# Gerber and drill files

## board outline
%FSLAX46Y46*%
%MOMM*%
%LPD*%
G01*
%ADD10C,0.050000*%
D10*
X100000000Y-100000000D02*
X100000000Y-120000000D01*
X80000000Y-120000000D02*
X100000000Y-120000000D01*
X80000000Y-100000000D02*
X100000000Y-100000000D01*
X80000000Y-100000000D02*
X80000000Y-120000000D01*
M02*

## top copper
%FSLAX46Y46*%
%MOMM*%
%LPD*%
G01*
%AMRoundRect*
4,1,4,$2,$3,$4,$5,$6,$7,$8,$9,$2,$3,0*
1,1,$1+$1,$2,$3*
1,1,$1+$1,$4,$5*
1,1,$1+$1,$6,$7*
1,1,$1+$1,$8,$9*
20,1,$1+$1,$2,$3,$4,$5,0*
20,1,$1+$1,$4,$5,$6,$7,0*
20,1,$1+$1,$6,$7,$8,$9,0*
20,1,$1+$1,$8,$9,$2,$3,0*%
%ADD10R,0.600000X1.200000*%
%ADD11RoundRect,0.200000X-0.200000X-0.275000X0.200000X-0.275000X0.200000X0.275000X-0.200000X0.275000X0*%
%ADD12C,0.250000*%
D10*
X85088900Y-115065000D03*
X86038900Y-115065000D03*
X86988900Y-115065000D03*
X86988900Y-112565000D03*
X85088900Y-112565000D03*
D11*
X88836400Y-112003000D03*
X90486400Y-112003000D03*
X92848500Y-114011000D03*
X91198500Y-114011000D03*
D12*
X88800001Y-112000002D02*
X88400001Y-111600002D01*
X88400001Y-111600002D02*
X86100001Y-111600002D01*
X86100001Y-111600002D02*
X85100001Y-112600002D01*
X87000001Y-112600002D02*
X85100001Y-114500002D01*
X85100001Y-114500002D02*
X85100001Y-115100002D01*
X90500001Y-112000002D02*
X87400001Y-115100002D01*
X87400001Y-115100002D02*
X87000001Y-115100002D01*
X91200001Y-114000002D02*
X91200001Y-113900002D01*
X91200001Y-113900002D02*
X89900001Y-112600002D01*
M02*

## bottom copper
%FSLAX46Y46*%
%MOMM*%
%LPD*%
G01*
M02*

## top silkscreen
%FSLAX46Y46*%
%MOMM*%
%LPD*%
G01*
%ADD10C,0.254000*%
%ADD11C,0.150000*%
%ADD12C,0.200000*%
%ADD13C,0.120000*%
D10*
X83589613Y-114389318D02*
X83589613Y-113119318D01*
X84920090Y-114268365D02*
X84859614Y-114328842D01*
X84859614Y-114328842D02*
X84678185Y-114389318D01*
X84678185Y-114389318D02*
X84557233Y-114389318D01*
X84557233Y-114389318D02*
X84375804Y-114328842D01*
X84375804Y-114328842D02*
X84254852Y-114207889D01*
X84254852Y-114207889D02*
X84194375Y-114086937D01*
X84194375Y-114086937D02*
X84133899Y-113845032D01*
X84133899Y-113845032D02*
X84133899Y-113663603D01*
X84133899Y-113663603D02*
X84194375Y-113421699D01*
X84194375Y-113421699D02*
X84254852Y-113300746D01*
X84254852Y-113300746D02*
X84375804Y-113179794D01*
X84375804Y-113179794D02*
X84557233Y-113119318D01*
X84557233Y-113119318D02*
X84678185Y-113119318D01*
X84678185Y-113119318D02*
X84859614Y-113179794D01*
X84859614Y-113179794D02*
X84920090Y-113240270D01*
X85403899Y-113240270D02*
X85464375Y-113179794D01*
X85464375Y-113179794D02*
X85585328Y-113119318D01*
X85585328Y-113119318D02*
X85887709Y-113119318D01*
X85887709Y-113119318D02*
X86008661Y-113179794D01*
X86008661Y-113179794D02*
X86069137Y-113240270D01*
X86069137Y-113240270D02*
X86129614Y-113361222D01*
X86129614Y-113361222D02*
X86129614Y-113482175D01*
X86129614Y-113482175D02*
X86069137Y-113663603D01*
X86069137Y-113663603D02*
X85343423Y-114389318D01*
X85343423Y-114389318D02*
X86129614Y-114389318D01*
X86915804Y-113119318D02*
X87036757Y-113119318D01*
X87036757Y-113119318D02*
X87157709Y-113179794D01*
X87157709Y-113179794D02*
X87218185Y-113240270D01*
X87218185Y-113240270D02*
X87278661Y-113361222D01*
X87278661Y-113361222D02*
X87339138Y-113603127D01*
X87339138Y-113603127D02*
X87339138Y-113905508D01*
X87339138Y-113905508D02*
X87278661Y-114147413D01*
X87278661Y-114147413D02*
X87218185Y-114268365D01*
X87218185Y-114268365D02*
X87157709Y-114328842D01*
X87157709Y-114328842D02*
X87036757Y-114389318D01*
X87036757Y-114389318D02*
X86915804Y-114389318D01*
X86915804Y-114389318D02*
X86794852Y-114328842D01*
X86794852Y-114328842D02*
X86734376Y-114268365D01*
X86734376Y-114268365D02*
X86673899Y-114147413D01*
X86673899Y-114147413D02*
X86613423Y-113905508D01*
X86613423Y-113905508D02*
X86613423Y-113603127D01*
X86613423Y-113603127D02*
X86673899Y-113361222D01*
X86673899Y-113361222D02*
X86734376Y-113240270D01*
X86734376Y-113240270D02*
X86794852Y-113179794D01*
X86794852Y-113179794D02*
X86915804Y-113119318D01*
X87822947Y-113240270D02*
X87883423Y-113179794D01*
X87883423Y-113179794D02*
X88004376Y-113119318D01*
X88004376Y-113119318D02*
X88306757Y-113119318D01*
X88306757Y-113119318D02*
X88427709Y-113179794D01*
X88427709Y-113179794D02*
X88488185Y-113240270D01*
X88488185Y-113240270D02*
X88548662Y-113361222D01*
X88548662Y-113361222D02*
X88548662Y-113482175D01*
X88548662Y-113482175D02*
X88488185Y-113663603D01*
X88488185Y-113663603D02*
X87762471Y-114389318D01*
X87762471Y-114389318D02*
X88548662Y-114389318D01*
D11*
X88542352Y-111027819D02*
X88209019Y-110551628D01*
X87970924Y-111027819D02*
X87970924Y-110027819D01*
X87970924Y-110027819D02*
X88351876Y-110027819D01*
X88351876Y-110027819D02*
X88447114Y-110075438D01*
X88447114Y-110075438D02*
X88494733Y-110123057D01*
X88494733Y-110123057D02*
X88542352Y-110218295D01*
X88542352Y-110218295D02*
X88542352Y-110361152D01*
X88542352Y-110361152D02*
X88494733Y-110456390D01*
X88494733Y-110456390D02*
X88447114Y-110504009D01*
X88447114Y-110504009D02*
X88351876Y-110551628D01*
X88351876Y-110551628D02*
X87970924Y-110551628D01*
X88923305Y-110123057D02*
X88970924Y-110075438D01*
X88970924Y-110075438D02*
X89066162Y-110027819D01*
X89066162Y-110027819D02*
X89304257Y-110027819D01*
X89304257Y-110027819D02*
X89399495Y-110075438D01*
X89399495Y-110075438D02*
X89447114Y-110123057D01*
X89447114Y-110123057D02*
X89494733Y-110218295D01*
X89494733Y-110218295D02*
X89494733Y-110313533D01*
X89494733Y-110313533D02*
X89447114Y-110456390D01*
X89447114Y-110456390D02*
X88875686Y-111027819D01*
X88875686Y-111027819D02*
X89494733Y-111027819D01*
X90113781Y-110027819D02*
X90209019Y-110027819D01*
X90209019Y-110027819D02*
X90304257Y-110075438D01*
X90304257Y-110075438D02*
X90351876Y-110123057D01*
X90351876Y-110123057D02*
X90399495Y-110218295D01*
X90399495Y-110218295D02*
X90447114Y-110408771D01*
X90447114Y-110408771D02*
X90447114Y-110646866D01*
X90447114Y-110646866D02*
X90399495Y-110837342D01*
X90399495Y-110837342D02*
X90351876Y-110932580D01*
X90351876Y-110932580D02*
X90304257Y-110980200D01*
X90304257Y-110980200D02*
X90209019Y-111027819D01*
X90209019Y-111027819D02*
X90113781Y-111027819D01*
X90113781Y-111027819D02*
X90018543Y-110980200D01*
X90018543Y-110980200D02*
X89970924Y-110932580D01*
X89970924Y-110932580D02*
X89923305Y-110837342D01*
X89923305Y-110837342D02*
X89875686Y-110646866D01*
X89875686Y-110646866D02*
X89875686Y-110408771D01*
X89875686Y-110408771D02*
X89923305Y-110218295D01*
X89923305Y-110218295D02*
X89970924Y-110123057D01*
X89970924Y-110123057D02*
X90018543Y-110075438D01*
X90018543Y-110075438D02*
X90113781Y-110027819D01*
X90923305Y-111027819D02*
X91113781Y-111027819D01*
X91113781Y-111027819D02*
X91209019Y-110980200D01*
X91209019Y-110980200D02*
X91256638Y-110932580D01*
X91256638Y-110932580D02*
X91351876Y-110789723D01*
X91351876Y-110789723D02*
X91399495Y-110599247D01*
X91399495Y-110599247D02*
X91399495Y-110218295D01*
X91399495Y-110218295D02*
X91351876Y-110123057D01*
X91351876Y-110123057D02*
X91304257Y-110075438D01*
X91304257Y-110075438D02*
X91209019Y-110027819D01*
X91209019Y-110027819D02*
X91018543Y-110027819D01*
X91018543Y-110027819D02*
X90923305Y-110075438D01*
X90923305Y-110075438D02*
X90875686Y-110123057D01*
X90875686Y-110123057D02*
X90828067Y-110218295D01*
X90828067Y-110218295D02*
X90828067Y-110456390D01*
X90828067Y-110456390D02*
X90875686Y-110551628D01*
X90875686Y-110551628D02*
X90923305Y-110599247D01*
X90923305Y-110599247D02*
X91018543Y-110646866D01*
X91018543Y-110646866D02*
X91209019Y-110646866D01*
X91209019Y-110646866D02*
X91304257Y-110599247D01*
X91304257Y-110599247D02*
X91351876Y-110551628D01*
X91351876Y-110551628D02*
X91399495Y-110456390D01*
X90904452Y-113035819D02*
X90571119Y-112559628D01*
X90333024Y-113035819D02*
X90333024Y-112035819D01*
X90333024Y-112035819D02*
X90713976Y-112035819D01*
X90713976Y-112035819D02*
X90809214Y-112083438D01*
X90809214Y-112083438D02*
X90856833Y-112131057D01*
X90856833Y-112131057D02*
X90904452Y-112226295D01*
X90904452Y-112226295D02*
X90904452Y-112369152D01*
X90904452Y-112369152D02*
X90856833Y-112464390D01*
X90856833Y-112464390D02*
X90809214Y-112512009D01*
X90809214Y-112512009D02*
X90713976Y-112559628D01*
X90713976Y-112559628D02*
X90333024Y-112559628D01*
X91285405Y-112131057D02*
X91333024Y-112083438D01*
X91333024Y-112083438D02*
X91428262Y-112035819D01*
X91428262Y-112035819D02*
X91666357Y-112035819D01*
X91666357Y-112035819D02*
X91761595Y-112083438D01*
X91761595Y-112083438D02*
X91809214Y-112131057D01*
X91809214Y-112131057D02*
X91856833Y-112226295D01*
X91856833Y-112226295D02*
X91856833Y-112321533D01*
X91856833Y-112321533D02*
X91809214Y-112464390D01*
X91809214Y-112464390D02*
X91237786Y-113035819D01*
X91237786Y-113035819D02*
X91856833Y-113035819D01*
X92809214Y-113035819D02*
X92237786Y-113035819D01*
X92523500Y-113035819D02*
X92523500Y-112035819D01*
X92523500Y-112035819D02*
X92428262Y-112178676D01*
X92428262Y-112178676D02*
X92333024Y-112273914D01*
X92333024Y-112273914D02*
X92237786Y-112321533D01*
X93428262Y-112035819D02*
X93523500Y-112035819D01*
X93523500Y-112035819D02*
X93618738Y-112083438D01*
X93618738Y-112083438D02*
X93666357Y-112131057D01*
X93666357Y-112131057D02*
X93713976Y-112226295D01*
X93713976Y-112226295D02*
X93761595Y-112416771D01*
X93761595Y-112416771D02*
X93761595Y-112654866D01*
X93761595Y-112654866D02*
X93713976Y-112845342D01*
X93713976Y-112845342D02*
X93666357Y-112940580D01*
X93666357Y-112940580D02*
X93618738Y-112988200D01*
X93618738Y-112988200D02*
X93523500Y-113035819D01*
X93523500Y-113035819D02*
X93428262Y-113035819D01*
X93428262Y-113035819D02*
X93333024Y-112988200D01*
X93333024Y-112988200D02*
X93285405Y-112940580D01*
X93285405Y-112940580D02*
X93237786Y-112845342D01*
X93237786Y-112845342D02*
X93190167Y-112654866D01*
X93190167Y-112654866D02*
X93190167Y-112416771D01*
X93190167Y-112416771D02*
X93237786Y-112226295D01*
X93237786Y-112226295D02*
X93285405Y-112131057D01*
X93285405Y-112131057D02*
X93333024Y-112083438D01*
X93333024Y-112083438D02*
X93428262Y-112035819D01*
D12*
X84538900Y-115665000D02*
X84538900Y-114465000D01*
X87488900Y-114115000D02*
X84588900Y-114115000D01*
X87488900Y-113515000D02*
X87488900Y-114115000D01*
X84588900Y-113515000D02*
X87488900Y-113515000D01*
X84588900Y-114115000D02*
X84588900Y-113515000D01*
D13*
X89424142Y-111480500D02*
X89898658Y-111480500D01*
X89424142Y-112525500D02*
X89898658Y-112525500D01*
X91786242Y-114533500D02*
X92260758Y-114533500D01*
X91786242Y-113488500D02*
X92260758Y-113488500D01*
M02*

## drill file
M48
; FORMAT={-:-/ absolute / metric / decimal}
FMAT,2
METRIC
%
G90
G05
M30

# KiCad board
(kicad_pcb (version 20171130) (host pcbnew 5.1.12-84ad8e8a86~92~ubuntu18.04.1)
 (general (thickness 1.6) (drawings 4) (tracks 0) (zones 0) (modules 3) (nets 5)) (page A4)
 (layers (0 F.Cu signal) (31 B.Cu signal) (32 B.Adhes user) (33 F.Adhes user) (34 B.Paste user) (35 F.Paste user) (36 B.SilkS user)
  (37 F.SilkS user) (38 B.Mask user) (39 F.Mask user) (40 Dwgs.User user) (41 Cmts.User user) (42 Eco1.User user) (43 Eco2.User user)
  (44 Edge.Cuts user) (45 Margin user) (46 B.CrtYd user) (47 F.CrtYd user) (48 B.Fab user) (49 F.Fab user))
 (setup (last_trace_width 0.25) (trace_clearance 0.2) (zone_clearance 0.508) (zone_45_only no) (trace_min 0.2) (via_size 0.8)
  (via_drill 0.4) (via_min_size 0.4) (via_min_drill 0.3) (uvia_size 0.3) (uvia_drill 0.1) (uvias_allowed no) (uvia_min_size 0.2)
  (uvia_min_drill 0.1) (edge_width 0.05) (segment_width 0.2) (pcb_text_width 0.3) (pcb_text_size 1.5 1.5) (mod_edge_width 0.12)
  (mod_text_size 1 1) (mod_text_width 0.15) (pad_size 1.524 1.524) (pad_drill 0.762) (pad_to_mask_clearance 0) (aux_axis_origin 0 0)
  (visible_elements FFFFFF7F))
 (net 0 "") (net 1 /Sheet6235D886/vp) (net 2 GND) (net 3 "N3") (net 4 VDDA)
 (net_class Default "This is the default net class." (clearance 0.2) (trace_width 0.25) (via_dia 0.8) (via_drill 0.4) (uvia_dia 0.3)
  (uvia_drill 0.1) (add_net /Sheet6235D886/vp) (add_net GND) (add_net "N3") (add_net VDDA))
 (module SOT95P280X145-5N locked (layer F.Cu) (at 86.038900 113.815000 90.000000)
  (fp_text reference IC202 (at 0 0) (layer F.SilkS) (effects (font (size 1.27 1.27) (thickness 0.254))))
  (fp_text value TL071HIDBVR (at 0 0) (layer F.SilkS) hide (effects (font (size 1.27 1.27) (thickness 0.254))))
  (fp_line (start -1.85 -1.5) (end -0.65 -1.5) (layer F.SilkS) (width 0.2))
  (fp_line (start -0.3 1.45) (end -0.3 -1.45) (layer F.SilkS) (width 0.2))
  (fp_line (start 0.3 1.45) (end -0.3 1.45) (layer F.SilkS) (width 0.2))
  (fp_line (start 0.3 -1.45) (end 0.3 1.45) (layer F.SilkS) (width 0.2))
  (fp_line (start -0.3 -1.45) (end 0.3 -1.45) (layer F.SilkS) (width 0.2))
  (pad 1 smd rect (at -1.25 -0.95 180.000000) (size 0.6 1.2) (layers F.Cu F.Mask F.Paste) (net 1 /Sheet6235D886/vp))
  (pad 2 smd rect (at -1.25 0 180.000000) (size 0.6 1.2) (layers F.Cu F.Mask F.Paste) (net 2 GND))
  (pad 3 smd rect (at -1.25 0.95 180.000000) (size 0.6 1.2) (layers F.Cu F.Mask F.Paste) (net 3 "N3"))
  (pad 4 smd rect (at 1.25 0.95 180.000000) (size 0.6 1.2) (layers F.Cu F.Mask F.Paste) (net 1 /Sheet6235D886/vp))
  (pad 5 smd rect (at 1.25 -0.95 180.000000) (size 0.6 1.2) (layers F.Cu F.Mask F.Paste) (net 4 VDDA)))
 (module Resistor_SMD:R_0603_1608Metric (layer F.Cu) (at 89.661400 112.003000)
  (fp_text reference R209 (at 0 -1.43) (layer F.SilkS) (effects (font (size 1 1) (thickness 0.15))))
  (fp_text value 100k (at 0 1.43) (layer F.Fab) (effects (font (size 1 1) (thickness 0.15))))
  (fp_line (start -0.237258 -0.5225) (end 0.237258 -0.5225) (layer F.SilkS) (width 0.12))
  (fp_line (start -0.237258 0.5225) (end 0.237258 0.5225) (layer F.SilkS) (width 0.12))
  (pad 1 smd roundrect (at -0.825 0) (size 0.8 0.95) (layers F.Cu F.Mask F.Paste) (roundrect_rratio 0.25) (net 4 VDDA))
  (pad 2 smd roundrect (at 0.825 0) (size 0.8 0.95) (layers F.Cu F.Mask F.Paste) (roundrect_rratio 0.25) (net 3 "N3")))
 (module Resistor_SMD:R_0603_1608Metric (layer F.Cu) (at 92.023500 114.011000)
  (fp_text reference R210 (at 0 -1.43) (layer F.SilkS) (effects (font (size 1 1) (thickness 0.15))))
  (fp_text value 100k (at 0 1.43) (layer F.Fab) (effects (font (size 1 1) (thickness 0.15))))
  (fp_line (start -0.237258 0.5225) (end 0.237258 0.5225) (layer F.SilkS) (width 0.12))
  (fp_line (start -0.237258 -0.5225) (end 0.237258 -0.5225) (layer F.SilkS) (width 0.12))
  (pad 2 smd roundrect (at 0.825 0) (size 0.8 0.95) (layers F.Cu F.Mask F.Paste) (roundrect_rratio 0.25) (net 2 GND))
  (pad 1 smd roundrect (at -0.825 0) (size 0.8 0.95) (layers F.Cu F.Mask F.Paste) (roundrect_rratio 0.25) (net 3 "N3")))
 (gr_line (start 100 100) (end 100 120) (layer Edge.Cuts) (width 0.05))
 (gr_line (start 80 120) (end 100 120) (layer Edge.Cuts) (width 0.05))
 (gr_line (start 80 100) (end 100 100) (layer Edge.Cuts) (width 0.05))
 (gr_line (start 80 100) (end 80 120) (layer Edge.Cuts) (width 0.05))
 (segment (start 88.800001 112.000002) (end 88.400001 111.600002) (width 0.250000) (layer F.Cu) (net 4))
 (segment (start 88.400001 111.600002) (end 86.100001 111.600002) (width 0.250000) (layer F.Cu) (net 4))
 (segment (start 86.100001 111.600002) (end 85.100001 112.600002) (width 0.250000) (layer F.Cu) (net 4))
 (segment (start 87.000001 112.600002) (end 85.100001 114.500002) (width 0.250000) (layer F.Cu) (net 1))
 (segment (start 85.100001 114.500002) (end 85.100001 115.100002) (width 0.250000) (layer F.Cu) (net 1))
 (segment (start 90.500001 112.000002) (end 87.400001 115.100002) (width 0.250000) (layer F.Cu) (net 3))
 (segment (start 87.400001 115.100002) (end 87.000001 115.100002) (width 0.250000) (layer F.Cu) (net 3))
 (segment (start 91.200001 114.000002) (end 91.200001 113.900002) (width 0.250000) (layer F.Cu) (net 3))
 (segment (start 91.200001 113.900002) (end 89.900001 112.600002) (width 0.250000) (layer F.Cu) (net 3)))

